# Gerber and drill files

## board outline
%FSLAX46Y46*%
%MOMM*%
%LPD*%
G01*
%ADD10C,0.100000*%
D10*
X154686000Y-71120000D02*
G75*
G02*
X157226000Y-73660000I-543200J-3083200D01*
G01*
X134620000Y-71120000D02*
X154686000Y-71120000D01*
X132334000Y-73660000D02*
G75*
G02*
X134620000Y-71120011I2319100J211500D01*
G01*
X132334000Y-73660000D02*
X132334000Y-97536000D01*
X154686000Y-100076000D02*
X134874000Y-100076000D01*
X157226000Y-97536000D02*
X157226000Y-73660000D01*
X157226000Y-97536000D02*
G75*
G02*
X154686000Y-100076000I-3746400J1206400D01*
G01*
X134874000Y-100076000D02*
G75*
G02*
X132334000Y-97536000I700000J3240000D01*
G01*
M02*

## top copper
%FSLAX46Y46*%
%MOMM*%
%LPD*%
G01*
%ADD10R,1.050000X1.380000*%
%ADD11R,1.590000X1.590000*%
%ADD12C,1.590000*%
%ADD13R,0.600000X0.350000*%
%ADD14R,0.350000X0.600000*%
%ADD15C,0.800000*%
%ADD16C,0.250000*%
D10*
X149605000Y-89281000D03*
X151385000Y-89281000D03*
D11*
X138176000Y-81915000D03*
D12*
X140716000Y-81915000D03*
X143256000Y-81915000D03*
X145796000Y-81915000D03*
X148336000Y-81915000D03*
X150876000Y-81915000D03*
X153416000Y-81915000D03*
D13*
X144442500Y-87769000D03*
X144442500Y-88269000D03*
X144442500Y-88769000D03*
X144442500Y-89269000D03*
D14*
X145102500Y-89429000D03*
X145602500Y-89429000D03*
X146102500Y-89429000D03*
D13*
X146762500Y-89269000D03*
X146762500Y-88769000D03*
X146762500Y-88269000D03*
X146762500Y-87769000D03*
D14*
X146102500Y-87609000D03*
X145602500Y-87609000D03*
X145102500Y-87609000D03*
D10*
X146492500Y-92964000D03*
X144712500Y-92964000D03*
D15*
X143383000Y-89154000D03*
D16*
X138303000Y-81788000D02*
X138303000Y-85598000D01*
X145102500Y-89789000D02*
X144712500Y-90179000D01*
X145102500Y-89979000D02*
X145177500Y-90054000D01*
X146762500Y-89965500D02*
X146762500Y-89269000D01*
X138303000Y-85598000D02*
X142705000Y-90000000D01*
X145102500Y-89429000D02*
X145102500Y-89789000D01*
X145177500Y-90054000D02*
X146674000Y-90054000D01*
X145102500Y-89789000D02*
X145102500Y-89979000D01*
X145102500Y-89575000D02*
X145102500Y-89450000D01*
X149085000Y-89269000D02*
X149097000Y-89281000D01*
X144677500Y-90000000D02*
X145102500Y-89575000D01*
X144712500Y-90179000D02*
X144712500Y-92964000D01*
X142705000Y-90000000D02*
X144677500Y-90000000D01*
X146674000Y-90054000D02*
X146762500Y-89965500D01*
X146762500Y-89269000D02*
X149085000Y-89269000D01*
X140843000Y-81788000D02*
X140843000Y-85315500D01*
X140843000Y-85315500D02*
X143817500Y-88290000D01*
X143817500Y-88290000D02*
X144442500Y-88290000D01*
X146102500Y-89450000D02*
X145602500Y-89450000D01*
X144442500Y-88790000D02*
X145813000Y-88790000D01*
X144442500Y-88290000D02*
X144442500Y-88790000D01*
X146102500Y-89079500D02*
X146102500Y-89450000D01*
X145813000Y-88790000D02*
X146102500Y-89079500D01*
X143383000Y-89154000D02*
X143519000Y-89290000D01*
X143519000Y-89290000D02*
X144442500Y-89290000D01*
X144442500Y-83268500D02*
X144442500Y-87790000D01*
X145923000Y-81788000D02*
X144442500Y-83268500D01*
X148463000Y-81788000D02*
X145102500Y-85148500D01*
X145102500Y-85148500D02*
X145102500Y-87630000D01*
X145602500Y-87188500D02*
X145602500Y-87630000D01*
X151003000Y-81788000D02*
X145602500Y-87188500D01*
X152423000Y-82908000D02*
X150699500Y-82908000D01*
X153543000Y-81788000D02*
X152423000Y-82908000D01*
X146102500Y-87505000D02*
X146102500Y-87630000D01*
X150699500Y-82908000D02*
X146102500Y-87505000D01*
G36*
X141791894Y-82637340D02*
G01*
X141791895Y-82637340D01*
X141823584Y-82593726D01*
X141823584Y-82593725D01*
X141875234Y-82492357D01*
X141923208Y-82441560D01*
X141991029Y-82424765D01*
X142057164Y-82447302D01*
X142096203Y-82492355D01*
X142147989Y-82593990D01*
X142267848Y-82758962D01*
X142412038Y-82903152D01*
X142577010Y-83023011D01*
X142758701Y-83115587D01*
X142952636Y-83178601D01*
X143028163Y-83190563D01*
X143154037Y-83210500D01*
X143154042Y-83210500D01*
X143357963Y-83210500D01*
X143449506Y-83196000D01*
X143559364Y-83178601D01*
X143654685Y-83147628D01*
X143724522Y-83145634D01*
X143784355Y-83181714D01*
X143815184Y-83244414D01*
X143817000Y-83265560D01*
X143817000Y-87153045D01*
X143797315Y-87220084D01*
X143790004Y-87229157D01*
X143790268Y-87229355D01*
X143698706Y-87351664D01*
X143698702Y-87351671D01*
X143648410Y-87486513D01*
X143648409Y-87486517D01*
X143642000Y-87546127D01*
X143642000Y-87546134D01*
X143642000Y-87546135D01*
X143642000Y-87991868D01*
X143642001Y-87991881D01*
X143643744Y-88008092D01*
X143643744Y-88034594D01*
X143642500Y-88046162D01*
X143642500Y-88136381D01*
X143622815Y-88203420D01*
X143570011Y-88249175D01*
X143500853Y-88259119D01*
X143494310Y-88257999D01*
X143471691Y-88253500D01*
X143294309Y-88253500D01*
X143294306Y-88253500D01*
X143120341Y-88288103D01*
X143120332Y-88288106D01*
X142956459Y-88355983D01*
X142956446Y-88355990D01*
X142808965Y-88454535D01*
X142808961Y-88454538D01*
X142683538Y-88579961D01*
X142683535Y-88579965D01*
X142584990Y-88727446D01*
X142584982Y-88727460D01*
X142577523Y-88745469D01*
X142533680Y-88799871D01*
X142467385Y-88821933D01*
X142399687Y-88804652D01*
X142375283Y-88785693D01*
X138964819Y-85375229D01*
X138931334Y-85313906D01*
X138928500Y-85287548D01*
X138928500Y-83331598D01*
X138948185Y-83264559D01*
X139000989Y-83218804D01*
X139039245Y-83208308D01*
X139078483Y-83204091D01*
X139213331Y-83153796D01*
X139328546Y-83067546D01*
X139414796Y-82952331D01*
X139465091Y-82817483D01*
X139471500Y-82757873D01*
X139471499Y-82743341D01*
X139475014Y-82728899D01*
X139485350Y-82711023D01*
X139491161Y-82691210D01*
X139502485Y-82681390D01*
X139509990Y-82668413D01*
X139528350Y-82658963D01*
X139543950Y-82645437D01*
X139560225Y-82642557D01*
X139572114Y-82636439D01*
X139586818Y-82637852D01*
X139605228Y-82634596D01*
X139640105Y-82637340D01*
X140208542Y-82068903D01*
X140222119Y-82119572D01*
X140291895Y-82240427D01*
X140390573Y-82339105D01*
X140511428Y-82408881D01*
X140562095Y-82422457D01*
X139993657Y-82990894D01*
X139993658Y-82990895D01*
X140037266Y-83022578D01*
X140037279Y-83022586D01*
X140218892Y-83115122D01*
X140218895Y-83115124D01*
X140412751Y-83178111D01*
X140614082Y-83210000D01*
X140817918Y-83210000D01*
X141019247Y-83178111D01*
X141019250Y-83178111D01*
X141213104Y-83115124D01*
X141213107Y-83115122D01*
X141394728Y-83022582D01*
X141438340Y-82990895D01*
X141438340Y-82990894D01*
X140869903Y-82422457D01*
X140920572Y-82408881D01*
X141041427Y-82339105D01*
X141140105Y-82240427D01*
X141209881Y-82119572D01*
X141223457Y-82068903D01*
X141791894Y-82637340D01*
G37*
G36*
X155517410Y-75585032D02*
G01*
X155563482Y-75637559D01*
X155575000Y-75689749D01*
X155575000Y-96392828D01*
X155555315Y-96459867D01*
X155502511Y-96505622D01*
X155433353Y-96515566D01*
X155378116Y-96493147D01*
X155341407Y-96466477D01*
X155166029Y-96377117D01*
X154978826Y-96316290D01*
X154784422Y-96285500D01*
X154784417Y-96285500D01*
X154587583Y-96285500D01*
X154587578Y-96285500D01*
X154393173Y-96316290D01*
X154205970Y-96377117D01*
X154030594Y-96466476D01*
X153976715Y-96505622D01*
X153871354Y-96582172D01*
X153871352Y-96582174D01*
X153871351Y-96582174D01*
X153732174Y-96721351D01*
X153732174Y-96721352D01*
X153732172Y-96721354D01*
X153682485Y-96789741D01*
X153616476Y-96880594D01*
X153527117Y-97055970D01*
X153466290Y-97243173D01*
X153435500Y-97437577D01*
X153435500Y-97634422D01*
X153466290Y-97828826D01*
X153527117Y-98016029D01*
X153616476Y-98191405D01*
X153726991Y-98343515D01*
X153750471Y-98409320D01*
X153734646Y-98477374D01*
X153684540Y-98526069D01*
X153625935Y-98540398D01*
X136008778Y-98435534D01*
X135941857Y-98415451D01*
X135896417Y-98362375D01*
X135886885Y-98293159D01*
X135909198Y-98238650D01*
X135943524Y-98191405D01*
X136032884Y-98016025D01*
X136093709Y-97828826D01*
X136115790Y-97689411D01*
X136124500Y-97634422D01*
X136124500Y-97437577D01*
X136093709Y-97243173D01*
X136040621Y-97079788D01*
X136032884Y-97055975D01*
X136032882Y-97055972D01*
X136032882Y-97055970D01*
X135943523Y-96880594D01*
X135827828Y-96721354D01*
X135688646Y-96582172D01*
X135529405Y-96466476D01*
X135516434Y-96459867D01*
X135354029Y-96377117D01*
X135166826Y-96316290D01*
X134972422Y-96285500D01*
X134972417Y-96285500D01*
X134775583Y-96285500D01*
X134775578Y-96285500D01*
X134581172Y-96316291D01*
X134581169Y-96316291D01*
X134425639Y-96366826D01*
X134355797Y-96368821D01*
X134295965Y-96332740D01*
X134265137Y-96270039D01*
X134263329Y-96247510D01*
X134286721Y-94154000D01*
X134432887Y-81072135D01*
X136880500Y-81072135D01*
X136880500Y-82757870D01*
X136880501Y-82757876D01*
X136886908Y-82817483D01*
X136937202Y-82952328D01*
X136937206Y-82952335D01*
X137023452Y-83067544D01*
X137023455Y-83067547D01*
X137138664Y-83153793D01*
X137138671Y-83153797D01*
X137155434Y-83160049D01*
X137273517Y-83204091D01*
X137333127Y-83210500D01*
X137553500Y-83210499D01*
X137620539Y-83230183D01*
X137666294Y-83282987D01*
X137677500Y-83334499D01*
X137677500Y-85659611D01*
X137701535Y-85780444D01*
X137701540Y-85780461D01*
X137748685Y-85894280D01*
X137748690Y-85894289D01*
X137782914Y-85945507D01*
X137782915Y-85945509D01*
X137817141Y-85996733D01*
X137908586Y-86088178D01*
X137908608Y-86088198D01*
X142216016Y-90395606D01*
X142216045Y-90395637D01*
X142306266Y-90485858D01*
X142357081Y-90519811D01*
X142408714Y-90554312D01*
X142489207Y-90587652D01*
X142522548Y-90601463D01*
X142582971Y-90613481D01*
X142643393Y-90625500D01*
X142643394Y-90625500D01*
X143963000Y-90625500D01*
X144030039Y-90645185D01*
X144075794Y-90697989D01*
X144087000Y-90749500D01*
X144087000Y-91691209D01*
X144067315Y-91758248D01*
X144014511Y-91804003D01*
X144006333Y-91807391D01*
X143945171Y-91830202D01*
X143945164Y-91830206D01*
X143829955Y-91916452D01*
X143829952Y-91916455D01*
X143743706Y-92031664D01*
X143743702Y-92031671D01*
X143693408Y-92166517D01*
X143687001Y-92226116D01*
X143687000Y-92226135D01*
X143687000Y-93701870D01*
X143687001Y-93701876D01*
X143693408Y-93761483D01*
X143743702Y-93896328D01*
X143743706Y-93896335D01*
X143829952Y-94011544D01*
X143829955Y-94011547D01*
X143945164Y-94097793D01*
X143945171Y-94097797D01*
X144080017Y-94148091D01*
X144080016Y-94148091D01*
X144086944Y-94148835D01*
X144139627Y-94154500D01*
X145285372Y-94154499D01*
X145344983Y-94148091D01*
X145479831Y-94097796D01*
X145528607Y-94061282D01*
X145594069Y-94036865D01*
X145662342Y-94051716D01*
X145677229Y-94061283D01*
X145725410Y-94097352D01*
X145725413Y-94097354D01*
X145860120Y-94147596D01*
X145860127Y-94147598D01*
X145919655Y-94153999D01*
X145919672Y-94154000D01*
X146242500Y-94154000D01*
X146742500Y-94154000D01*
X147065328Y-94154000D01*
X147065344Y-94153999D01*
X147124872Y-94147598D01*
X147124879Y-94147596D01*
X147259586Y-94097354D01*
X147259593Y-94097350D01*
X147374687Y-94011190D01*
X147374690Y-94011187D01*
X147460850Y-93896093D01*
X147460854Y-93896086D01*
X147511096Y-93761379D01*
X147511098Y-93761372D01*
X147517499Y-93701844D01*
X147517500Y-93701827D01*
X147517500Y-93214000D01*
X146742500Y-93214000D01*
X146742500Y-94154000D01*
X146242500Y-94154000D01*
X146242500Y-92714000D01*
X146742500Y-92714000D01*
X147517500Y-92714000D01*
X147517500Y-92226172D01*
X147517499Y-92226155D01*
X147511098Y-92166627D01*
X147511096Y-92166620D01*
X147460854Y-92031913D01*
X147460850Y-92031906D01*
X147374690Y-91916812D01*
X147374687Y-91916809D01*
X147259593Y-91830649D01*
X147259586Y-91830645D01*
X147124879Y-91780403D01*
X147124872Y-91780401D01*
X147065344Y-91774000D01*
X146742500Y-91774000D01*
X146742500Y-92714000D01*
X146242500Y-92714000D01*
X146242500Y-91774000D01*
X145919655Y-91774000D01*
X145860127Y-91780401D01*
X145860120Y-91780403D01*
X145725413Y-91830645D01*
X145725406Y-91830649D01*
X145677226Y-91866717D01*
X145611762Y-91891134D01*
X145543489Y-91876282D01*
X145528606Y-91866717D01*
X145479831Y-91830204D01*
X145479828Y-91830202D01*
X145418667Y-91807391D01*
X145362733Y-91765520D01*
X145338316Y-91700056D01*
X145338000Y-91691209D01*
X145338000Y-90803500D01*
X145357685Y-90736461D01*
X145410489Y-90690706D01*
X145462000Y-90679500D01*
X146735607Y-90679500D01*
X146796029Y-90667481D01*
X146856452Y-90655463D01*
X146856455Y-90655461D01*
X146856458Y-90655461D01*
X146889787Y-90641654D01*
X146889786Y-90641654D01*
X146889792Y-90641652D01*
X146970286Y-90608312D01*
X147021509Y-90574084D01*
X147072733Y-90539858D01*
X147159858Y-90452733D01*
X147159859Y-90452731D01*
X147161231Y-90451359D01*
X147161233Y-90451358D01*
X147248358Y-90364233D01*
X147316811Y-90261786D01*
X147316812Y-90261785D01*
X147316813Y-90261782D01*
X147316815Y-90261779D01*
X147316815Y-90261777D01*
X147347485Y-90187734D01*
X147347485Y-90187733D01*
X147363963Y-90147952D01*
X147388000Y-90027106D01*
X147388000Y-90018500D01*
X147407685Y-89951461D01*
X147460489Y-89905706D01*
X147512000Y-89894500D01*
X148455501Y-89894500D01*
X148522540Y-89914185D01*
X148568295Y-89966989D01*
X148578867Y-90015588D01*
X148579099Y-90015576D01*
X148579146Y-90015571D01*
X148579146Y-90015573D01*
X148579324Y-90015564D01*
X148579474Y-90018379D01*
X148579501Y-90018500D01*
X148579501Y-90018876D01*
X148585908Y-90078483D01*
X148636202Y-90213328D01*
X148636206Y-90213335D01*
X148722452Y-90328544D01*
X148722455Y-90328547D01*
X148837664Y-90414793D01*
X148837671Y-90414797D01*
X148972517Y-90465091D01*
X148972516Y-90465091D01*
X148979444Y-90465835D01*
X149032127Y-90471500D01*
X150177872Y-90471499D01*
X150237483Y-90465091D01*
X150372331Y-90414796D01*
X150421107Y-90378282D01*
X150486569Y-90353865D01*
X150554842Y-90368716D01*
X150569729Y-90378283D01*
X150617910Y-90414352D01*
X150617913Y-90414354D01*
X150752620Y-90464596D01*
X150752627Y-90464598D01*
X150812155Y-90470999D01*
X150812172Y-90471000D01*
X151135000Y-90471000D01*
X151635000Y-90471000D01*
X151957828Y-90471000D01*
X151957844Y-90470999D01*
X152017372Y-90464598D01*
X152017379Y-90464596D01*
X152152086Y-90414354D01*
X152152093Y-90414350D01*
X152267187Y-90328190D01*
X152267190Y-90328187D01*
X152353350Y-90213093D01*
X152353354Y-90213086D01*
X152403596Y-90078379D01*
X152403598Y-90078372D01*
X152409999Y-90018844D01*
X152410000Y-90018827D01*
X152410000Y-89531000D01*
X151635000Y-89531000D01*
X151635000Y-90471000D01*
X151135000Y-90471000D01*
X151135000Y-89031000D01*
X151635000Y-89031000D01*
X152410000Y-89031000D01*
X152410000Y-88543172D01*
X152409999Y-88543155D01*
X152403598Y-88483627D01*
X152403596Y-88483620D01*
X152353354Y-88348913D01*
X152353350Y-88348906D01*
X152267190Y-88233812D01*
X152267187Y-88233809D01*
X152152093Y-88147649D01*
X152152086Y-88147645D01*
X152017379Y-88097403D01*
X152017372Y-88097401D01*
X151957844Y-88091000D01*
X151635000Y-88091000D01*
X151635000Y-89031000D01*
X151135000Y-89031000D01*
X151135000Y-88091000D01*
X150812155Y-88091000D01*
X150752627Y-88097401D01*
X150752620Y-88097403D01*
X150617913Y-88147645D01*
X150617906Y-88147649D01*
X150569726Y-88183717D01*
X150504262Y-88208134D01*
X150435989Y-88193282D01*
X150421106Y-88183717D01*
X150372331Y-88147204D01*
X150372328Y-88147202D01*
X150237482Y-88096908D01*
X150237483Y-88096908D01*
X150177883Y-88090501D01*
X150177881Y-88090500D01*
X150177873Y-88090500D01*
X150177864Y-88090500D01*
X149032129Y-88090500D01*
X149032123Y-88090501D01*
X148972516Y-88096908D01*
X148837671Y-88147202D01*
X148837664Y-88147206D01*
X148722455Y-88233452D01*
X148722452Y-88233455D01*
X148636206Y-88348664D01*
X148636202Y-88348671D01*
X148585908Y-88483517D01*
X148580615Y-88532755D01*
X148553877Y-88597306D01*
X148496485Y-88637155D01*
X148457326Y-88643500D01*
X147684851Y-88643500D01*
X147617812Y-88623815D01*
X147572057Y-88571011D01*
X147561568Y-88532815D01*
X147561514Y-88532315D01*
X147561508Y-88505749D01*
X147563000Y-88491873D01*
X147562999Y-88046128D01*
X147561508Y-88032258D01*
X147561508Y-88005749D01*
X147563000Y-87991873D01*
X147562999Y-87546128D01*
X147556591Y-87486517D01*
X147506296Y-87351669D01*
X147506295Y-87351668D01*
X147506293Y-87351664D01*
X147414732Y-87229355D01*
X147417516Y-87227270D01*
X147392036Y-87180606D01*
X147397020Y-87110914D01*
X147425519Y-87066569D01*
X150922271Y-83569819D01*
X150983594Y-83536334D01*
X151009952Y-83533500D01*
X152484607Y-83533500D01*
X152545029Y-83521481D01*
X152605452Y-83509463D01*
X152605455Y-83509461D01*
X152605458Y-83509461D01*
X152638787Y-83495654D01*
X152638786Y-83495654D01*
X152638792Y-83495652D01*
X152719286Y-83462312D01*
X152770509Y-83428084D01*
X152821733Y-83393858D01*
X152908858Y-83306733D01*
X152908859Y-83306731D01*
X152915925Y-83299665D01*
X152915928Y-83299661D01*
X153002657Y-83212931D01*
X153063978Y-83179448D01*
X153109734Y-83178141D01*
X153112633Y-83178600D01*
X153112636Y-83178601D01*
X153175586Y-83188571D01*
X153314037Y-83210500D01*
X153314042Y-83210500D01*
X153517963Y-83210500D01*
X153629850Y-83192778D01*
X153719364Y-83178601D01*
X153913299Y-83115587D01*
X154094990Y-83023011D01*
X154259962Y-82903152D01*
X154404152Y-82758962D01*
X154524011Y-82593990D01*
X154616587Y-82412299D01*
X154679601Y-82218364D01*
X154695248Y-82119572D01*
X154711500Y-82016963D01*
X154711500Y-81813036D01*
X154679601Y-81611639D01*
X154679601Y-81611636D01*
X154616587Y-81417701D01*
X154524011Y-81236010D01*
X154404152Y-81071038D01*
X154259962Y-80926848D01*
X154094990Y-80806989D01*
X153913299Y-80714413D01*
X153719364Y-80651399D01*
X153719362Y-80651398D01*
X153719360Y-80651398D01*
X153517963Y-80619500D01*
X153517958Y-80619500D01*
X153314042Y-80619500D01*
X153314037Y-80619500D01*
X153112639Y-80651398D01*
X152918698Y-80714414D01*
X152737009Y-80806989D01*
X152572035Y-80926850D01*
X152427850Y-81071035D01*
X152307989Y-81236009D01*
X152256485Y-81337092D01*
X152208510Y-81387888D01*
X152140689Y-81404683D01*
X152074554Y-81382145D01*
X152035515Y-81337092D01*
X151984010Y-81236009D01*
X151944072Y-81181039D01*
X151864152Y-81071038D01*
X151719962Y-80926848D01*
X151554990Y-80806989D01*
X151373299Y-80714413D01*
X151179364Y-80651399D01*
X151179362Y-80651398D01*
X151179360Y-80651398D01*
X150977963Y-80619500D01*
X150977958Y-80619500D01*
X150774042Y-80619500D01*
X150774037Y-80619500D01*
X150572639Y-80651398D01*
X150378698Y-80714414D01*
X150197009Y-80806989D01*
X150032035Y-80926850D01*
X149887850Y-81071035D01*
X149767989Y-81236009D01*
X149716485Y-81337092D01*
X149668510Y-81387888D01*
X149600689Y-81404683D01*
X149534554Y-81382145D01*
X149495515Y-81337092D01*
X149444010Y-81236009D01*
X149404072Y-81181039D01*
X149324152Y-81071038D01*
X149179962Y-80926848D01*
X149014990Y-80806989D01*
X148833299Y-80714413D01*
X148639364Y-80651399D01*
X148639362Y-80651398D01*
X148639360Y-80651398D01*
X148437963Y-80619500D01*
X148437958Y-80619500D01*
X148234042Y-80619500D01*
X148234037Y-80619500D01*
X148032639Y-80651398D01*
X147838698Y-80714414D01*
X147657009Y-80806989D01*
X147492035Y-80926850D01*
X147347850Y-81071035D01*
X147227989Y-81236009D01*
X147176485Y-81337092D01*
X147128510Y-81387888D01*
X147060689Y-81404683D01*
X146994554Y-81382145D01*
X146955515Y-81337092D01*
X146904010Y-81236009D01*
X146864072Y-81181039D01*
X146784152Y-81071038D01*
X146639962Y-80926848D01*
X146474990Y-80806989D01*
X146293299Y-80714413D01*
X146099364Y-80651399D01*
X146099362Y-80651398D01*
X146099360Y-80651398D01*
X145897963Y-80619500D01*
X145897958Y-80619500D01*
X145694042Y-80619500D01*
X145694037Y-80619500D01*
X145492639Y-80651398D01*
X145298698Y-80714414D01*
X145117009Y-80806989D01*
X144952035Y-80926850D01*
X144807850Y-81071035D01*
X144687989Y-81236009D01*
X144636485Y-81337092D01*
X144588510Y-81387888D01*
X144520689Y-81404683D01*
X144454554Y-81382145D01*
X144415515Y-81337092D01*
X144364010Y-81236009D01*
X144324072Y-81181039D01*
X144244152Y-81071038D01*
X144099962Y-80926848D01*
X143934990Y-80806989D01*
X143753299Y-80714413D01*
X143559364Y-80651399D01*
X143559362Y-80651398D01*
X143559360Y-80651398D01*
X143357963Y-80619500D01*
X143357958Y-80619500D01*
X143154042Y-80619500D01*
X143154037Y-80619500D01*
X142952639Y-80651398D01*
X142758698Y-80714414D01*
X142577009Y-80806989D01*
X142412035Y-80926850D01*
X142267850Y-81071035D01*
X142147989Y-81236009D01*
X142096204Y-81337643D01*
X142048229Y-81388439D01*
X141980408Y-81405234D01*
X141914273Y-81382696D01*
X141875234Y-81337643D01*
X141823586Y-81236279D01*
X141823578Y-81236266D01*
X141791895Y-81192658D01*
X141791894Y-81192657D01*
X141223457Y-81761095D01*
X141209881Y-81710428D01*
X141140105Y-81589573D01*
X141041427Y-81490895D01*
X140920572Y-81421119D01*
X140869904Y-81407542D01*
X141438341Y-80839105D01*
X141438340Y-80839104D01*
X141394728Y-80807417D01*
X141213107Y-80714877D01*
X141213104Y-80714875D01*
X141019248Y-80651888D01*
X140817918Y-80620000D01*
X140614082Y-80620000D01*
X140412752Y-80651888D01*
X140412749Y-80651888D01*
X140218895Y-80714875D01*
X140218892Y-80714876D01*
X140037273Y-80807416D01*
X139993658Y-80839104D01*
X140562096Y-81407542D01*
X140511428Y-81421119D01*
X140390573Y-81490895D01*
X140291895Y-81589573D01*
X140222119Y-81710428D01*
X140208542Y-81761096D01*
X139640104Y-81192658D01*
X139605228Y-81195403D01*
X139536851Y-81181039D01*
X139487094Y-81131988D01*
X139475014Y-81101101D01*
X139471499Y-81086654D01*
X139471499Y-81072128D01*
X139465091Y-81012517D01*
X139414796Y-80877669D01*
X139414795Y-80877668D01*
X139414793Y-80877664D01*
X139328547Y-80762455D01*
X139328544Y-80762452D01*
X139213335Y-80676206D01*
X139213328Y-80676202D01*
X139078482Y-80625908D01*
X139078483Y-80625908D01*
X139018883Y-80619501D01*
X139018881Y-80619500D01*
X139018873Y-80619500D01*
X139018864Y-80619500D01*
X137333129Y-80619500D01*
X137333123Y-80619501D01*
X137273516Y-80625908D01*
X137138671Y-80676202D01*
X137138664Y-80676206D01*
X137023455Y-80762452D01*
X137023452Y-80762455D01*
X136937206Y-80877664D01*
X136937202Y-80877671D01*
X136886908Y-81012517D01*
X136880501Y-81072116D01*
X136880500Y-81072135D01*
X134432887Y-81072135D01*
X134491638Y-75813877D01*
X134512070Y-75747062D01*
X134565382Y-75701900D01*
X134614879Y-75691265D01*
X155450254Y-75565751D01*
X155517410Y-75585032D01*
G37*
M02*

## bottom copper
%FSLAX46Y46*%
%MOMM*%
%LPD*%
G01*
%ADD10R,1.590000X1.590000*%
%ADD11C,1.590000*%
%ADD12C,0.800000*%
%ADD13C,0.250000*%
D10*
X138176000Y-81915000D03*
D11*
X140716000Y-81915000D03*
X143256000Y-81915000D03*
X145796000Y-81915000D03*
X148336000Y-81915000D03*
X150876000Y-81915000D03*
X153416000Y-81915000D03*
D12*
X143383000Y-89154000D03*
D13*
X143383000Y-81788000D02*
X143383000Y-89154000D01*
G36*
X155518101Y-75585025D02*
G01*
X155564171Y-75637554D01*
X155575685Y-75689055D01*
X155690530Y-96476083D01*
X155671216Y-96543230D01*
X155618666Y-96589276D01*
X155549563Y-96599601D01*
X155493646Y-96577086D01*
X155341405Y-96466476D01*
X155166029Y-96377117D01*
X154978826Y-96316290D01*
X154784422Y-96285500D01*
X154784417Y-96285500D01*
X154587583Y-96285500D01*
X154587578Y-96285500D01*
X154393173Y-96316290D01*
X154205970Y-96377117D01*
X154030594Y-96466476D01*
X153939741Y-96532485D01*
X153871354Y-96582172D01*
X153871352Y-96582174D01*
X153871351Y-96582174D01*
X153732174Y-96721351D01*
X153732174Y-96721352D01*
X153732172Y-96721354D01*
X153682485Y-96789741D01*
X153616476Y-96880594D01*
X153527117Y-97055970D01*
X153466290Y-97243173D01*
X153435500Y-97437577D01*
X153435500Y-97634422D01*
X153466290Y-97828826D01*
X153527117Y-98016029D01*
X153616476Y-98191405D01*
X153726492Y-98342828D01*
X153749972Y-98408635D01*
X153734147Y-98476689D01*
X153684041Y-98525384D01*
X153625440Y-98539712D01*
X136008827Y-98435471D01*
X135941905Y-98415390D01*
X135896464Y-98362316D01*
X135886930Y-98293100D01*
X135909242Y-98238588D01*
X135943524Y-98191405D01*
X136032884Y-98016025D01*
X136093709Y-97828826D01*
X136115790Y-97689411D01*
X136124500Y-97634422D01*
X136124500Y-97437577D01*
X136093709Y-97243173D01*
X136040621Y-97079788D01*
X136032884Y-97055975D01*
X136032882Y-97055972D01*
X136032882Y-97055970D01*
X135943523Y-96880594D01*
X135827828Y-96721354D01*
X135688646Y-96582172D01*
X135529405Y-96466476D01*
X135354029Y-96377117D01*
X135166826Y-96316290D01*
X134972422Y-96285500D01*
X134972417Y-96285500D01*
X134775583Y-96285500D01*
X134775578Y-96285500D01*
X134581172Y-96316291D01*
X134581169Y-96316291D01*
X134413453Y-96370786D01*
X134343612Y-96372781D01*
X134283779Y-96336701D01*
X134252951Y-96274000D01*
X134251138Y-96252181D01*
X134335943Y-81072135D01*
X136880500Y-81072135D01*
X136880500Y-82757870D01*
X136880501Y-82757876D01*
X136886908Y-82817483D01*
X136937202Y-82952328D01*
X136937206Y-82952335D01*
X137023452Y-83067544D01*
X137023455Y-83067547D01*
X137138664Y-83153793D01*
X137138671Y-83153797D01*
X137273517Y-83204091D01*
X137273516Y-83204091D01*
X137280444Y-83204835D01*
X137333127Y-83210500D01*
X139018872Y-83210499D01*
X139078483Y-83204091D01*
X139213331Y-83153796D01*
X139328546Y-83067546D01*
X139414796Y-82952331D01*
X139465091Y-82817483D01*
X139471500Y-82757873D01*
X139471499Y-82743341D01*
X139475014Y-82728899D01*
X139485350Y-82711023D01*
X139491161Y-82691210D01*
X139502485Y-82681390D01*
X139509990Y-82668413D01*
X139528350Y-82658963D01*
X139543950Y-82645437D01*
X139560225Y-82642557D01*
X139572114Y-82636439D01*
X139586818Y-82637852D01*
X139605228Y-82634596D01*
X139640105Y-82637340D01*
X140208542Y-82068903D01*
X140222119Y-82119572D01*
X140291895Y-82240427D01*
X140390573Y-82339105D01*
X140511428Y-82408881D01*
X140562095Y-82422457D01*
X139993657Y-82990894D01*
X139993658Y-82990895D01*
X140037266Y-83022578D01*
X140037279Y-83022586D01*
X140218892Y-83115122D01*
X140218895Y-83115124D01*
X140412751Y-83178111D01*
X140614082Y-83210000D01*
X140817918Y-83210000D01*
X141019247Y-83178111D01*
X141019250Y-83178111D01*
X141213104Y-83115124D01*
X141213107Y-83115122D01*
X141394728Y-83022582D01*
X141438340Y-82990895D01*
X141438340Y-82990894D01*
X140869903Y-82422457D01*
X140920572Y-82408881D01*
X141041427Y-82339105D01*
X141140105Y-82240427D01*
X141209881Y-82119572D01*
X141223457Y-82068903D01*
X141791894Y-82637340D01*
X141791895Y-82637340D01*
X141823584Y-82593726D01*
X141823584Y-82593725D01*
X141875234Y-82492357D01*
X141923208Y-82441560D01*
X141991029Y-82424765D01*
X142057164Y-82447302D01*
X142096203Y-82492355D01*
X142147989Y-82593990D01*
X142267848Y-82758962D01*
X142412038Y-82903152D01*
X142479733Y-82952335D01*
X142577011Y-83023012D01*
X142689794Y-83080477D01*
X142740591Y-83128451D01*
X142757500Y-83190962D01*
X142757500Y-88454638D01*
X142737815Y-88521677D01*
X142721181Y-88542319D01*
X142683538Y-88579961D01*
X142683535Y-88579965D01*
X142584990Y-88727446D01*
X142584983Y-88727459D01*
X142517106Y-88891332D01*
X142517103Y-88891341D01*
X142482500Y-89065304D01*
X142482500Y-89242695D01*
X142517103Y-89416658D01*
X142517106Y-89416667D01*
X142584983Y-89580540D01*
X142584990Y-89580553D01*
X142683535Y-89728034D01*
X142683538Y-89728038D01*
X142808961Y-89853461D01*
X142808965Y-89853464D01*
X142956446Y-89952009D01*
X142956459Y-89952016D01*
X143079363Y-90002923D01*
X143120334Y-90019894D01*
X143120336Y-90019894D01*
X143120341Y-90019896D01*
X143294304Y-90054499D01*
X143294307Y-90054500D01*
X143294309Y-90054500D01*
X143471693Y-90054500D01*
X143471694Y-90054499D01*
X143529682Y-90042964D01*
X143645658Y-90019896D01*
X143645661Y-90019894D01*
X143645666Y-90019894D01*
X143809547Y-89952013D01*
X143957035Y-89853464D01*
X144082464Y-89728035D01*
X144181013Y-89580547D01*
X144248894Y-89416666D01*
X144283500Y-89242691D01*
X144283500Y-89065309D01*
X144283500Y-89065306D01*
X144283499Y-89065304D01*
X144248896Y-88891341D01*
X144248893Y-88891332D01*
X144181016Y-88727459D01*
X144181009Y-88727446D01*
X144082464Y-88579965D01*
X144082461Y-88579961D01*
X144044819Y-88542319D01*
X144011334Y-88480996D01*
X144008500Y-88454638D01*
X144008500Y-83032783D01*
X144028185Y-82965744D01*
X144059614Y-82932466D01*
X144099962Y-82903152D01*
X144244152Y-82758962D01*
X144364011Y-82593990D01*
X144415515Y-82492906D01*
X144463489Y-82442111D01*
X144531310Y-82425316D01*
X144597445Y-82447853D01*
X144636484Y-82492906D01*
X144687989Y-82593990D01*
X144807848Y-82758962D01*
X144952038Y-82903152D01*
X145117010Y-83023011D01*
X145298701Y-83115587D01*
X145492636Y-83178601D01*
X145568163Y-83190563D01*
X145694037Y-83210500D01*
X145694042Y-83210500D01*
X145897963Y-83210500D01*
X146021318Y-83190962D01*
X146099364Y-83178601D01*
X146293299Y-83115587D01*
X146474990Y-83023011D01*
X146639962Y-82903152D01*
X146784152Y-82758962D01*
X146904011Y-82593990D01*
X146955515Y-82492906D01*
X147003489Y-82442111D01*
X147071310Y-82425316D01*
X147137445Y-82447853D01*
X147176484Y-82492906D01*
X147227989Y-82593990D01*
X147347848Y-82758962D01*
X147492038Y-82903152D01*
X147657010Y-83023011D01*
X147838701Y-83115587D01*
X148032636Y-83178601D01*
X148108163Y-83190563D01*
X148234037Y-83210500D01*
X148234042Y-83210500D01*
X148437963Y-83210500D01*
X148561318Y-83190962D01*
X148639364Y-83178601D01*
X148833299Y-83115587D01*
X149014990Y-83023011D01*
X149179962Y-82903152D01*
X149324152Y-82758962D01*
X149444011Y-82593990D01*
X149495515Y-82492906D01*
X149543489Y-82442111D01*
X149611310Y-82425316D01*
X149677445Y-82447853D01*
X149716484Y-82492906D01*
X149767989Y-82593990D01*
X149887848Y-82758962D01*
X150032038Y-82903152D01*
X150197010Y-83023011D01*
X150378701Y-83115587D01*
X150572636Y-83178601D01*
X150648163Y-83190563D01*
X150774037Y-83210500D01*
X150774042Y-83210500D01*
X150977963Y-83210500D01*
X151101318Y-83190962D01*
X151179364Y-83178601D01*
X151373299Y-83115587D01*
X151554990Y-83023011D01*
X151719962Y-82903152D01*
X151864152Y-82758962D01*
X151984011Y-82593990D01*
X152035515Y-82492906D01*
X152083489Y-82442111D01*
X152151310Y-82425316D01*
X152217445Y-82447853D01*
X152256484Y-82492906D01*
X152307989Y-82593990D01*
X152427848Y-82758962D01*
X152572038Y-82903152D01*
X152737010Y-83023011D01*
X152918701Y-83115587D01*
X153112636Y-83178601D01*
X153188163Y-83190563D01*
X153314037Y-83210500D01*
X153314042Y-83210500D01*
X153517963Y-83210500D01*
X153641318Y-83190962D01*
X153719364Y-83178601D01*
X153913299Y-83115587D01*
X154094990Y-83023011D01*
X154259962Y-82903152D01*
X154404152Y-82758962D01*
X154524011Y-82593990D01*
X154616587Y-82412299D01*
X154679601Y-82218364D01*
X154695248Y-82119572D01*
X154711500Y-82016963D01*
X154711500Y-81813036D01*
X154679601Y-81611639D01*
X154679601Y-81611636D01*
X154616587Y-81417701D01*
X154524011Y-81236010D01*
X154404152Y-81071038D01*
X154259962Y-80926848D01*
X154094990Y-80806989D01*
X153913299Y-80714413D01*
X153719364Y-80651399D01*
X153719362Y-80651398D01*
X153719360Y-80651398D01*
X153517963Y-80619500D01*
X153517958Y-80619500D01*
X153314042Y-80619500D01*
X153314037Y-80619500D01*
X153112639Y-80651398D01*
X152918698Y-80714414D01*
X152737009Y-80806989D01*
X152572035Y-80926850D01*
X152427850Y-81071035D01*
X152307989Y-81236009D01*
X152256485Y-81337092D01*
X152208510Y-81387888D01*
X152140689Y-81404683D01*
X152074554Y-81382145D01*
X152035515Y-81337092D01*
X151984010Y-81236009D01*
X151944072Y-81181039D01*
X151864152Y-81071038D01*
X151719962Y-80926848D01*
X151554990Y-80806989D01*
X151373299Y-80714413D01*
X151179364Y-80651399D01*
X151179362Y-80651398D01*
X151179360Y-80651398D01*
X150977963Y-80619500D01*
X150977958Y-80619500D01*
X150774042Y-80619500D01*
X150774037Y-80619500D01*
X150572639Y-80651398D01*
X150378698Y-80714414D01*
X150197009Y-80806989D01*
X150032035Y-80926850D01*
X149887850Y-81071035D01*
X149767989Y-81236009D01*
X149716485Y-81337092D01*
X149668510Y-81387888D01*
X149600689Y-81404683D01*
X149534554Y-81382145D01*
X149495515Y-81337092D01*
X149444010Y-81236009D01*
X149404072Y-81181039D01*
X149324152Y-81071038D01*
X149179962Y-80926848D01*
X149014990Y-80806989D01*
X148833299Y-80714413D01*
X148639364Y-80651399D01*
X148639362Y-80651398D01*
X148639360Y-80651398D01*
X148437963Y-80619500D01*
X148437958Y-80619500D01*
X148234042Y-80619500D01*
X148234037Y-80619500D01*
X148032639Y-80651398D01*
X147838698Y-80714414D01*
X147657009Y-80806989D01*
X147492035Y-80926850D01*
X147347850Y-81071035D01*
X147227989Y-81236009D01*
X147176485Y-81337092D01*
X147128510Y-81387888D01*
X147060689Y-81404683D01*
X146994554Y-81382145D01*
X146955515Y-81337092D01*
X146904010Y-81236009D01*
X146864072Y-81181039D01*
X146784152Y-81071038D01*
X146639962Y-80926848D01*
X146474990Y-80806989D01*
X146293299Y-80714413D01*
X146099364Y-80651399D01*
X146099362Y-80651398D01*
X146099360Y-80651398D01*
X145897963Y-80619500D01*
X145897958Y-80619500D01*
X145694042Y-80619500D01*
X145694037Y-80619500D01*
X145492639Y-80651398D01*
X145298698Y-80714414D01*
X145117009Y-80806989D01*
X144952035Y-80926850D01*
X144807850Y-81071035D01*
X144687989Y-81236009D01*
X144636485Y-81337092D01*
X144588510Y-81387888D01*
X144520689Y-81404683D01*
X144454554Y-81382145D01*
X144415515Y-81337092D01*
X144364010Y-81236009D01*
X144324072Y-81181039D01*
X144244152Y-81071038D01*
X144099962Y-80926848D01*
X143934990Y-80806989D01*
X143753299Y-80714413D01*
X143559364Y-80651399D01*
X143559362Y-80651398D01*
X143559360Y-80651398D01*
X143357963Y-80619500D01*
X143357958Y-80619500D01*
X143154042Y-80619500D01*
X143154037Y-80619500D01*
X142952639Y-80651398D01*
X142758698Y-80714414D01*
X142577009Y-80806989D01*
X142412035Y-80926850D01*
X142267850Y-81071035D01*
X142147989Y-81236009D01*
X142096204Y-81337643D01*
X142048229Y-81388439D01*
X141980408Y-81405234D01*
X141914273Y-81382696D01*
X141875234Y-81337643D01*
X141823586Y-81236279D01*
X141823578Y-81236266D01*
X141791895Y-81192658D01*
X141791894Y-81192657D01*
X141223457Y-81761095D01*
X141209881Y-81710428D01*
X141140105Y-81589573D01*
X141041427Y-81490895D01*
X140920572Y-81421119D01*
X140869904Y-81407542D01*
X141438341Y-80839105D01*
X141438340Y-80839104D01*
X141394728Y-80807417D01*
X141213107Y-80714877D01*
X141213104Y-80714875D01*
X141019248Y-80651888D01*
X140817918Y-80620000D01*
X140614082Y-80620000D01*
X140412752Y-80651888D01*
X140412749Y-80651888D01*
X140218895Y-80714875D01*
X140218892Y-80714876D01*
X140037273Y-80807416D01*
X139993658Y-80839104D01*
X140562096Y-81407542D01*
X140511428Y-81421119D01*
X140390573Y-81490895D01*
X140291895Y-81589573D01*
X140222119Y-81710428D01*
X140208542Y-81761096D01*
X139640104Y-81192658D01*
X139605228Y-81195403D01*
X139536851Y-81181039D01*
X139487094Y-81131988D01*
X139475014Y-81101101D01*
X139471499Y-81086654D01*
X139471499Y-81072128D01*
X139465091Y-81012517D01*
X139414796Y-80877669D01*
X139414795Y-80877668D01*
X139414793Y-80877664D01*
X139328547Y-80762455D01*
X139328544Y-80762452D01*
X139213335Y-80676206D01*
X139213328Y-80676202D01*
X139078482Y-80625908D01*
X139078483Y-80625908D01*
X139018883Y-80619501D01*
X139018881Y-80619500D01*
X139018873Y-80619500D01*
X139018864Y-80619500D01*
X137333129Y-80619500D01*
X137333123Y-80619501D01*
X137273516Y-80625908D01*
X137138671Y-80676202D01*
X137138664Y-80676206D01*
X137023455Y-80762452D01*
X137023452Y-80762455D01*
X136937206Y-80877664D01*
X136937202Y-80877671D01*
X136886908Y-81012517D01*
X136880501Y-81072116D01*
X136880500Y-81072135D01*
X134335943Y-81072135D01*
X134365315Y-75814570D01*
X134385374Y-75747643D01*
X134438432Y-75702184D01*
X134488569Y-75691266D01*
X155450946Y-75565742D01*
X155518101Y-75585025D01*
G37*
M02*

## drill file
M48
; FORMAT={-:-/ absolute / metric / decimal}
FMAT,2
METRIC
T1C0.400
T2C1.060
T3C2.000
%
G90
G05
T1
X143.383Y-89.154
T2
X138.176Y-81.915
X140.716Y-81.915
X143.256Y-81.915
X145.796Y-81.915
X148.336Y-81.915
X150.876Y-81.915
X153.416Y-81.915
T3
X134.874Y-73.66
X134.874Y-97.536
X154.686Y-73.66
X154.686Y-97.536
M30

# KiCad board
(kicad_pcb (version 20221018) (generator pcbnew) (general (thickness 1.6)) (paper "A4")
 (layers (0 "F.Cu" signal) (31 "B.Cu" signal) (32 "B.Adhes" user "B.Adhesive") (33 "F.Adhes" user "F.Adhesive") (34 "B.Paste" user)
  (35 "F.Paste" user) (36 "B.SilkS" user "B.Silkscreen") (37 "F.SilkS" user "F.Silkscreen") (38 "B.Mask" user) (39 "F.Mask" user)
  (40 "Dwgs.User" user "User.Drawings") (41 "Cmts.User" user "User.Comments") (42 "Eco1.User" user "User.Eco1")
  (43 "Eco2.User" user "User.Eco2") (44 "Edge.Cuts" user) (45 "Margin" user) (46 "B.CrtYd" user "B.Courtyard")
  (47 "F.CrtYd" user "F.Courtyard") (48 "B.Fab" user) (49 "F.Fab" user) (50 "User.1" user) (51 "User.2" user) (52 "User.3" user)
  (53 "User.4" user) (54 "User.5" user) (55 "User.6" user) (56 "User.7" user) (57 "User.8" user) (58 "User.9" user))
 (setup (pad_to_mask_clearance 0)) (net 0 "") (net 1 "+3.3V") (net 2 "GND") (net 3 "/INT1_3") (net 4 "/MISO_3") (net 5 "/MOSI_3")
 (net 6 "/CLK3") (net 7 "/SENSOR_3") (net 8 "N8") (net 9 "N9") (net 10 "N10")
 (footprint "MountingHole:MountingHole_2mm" (layer "F.Cu") (at 134.874 97.536)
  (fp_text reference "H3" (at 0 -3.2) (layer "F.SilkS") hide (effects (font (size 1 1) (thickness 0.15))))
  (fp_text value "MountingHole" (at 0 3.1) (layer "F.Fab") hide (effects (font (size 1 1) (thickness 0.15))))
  (pad "" np_thru_hole circle (at 0 0) (size 2 2) (drill 2) (layers "*.Cu" "*.Mask")))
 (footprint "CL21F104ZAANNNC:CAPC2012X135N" (layer "F.Cu") (at 150.495 89.281)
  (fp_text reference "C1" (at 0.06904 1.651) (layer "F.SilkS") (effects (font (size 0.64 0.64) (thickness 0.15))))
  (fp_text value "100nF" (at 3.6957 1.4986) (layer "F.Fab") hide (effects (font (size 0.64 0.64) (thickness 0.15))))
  (pad "1" smd rect (at -0.89 0) (size 1.05 1.38) (layers "F.Cu" "F.Paste" "F.Mask") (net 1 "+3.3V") (solder_mask_margin 0.102))
  (pad "2" smd rect (at 0.89 0) (size 1.05 1.38) (layers "F.Cu" "F.Paste" "F.Mask") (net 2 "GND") (solder_mask_margin 0.102)))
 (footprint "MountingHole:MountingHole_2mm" (layer "F.Cu") (at 154.686 73.66)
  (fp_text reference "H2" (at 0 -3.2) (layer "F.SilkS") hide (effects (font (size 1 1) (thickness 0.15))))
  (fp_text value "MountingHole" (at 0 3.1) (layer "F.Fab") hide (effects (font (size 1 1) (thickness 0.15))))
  (pad "" np_thru_hole circle (at 0 0) (size 2 2) (drill 2) (layers "*.Cu" "*.Mask")))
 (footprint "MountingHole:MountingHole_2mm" (layer "F.Cu") (at 134.874 73.66)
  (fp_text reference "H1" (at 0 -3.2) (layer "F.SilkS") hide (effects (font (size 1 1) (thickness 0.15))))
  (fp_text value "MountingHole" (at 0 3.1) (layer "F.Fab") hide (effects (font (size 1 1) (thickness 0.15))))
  (pad "" np_thru_hole circle (at 0 0) (size 2 2) (drill 2) (layers "*.Cu" "*.Mask")))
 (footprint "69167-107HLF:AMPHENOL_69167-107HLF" (layer "F.Cu") (at 145.796 81.915)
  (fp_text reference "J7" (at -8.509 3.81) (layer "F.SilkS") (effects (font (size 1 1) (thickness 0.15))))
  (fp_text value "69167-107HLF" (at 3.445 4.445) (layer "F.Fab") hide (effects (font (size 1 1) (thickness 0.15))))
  (pad "01" thru_hole rect (at -7.62 0) (size 1.59 1.59) (drill 1.06) (layers "*.Cu" "*.Mask") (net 1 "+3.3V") (solder_mask_margin 0.102))
  (pad "02" thru_hole circle (at -5.08 0) (size 1.59 1.59) (drill 1.06) (layers "*.Cu" "*.Mask") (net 2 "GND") (solder_mask_margin 0.102))
  (pad "03" thru_hole circle (at -2.54 0) (size 1.59 1.59) (drill 1.06) (layers "*.Cu" "*.Mask") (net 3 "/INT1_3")
   (solder_mask_margin 0.102))
  (pad "04" thru_hole circle (at 0 0) (size 1.59 1.59) (drill 1.06) (layers "*.Cu" "*.Mask") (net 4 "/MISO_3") (solder_mask_margin 0.102))
  (pad "05" thru_hole circle (at 2.54 0) (size 1.59 1.59) (drill 1.06) (layers "*.Cu" "*.Mask") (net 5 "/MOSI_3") (solder_mask_margin 0.102))
  (pad "06" thru_hole circle (at 5.08 0) (size 1.59 1.59) (drill 1.06) (layers "*.Cu" "*.Mask") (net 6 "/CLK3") (solder_mask_margin 0.102))
  (pad "07" thru_hole circle (at 7.62 0) (size 1.59 1.59) (drill 1.06) (layers "*.Cu" "*.Mask") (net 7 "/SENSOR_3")
   (solder_mask_margin 0.102)))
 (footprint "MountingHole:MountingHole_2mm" (layer "F.Cu") (at 154.686 97.536)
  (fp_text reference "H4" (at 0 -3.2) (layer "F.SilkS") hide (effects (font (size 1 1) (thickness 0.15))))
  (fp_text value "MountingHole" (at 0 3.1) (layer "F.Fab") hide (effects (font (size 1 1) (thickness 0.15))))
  (pad "" np_thru_hole circle (at 0 0) (size 2 2) (drill 2) (layers "*.Cu" "*.Mask")))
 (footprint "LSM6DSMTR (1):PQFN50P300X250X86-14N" (layer "F.Cu") (at 145.6025 88.519)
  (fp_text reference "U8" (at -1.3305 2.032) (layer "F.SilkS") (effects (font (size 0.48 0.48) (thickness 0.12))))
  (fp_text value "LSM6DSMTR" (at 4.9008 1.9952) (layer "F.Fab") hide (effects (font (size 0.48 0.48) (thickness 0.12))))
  (pad "1" smd rect (at -1.16 -0.75) (size 0.6 0.35) (layers "F.Cu" "F.Paste" "F.Mask") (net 4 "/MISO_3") (solder_mask_margin 0.102))
  (pad "2" smd rect (at -1.16 -0.25) (size 0.6 0.35) (layers "F.Cu" "F.Paste" "F.Mask") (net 2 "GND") (solder_mask_margin 0.102))
  (pad "3" smd rect (at -1.16 0.25) (size 0.6 0.35) (layers "F.Cu" "F.Paste" "F.Mask") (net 2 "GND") (solder_mask_margin 0.102))
  (pad "4" smd rect (at -1.16 0.75) (size 0.6 0.35) (layers "F.Cu" "F.Paste" "F.Mask") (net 3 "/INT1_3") (solder_mask_margin 0.102))
  (pad "5" smd rect (at -0.5 0.91 90) (size 0.6 0.35) (layers "F.Cu" "F.Paste" "F.Mask") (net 1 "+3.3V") (solder_mask_margin 0.102))
  (pad "6" smd rect (at 0 0.91 90) (size 0.6 0.35) (layers "F.Cu" "F.Paste" "F.Mask") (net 2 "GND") (solder_mask_margin 0.102))
  (pad "7" smd rect (at 0.5 0.91 90) (size 0.6 0.35) (layers "F.Cu" "F.Paste" "F.Mask") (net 2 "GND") (solder_mask_margin 0.102))
  (pad "8" smd rect (at 1.16 0.75) (size 0.6 0.35) (layers "F.Cu" "F.Paste" "F.Mask") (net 1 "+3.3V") (solder_mask_margin 0.102))
  (pad "9" smd rect (at 1.16 0.25) (size 0.6 0.35) (layers "F.Cu" "F.Paste" "F.Mask") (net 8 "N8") (solder_mask_margin 0.102))
  (pad "10" smd rect (at 1.16 -0.25) (size 0.6 0.35) (layers "F.Cu" "F.Paste" "F.Mask") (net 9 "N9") (solder_mask_margin 0.102))
  (pad "11" smd rect (at 1.16 -0.75) (size 0.6 0.35) (layers "F.Cu" "F.Paste" "F.Mask") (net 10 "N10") (solder_mask_margin 0.102))
  (pad "12" smd rect (at 0.5 -0.91 90) (size 0.6 0.35) (layers "F.Cu" "F.Paste" "F.Mask") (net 7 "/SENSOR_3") (solder_mask_margin 0.102))
  (pad "13" smd rect (at 0 -0.91 90) (size 0.6 0.35) (layers "F.Cu" "F.Paste" "F.Mask") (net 6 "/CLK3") (solder_mask_margin 0.102))
  (pad "14" smd rect (at -0.5 -0.91 90) (size 0.6 0.35) (layers "F.Cu" "F.Paste" "F.Mask") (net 5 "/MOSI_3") (solder_mask_margin 0.102)))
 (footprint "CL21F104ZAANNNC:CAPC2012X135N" (layer "F.Cu") (at 145.6025 92.964 180)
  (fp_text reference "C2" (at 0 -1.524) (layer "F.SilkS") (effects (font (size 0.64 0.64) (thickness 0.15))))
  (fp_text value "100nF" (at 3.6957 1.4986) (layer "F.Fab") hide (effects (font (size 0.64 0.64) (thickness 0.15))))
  (pad "1" smd rect (at -0.89 0 180) (size 1.05 1.38) (layers "F.Cu" "F.Paste" "F.Mask") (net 2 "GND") (solder_mask_margin 0.102))
  (pad "2" smd rect (at 0.89 0 180) (size 1.05 1.38) (layers "F.Cu" "F.Paste" "F.Mask") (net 1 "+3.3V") (solder_mask_margin 0.102)))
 (gr_arc (start 154.686 71.12) (mid 156.356529 71.989471) (end 157.226 73.66) (stroke (width 0.1) (type default)) (layer "Edge.Cuts"))
 (gr_line (start 134.62 71.12) (end 154.686 71.12) (stroke (width 0.1) (type default)) (layer "Edge.Cuts"))
 (gr_arc (start 132.334 73.66) (mid 132.922178 71.89066) (end 134.62 71.12) (stroke (width 0.1) (type default)) (layer "Edge.Cuts"))
 (gr_line (start 132.334 73.66) (end 132.334 97.536) (stroke (width 0.1) (type default)) (layer "Edge.Cuts"))
 (gr_line (start 154.686 100.076) (end 134.874 100.076) (stroke (width 0.1) (type default)) (layer "Edge.Cuts"))
 (gr_line (start 157.226 97.536) (end 157.226 73.66) (stroke (width 0.1) (type default)) (layer "Edge.Cuts"))
 (gr_arc (start 157.226 97.536) (mid 156.262666 99.112666) (end 154.686 100.076) (stroke (width 0.1) (type default)) (layer "Edge.Cuts"))
 (gr_arc (start 134.874 100.076) (mid 133.230114 99.179886) (end 132.334 97.536) (stroke (width 0.1) (type default)) (layer "Edge.Cuts"))
 (segment (start 138.303 81.788) (end 138.303 85.598) (width 0.25) (layer "F.Cu") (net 1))
 (segment (start 145.1025 89.789) (end 144.7125 90.179) (width 0.25) (layer "F.Cu") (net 1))
 (segment (start 145.1025 89.979) (end 145.1775 90.054) (width 0.25) (layer "F.Cu") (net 1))
 (segment (start 146.7625 89.9655) (end 146.7625 89.269) (width 0.25) (layer "F.Cu") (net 1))
 (segment (start 138.303 85.598) (end 142.705 90) (width 0.25) (layer "F.Cu") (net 1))
 (segment (start 145.1025 89.429) (end 145.1025 89.789) (width 0.25) (layer "F.Cu") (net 1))
 (segment (start 145.1775 90.054) (end 146.674 90.054) (width 0.25) (layer "F.Cu") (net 1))
 (segment (start 145.1025 89.789) (end 145.1025 89.979) (width 0.25) (layer "F.Cu") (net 1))
 (segment (start 145.1025 89.575) (end 145.1025 89.45) (width 0.25) (layer "F.Cu") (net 1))
 (segment (start 149.085 89.269) (end 149.097 89.281) (width 0.25) (layer "F.Cu") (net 1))
 (segment (start 144.6775 90) (end 145.1025 89.575) (width 0.25) (layer "F.Cu") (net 1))
 (segment (start 144.7125 90.179) (end 144.7125 92.964) (width 0.25) (layer "F.Cu") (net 1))
 (segment (start 142.705 90) (end 144.6775 90) (width 0.25) (layer "F.Cu") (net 1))
 (segment (start 146.674 90.054) (end 146.7625 89.9655) (width 0.25) (layer "F.Cu") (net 1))
 (segment (start 146.7625 89.269) (end 149.085 89.269) (width 0.25) (layer "F.Cu") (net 1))
 (segment (start 140.843 81.788) (end 140.843 85.3155) (width 0.25) (layer "F.Cu") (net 2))
 (segment (start 140.843 85.3155) (end 143.8175 88.29) (width 0.25) (layer "F.Cu") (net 2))
 (segment (start 143.8175 88.29) (end 144.4425 88.29) (width 0.25) (layer "F.Cu") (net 2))
 (segment (start 146.1025 89.45) (end 145.6025 89.45) (width 0.25) (layer "F.Cu") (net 2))
 (segment (start 144.4425 88.79) (end 145.813 88.79) (width 0.25) (layer "F.Cu") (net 2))
 (segment (start 144.4425 88.29) (end 144.4425 88.79) (width 0.25) (layer "F.Cu") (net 2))
 (segment (start 146.1025 89.0795) (end 146.1025 89.45) (width 0.25) (layer "F.Cu") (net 2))
 (segment (start 145.813 88.79) (end 146.1025 89.0795) (width 0.25) (layer "F.Cu") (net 2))
 (segment (start 143.383 89.154) (end 143.519 89.29) (width 0.25) (layer "F.Cu") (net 3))
 (segment (start 143.519 89.29) (end 144.4425 89.29) (width 0.25) (layer "F.Cu") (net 3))
 (via (at 143.383 89.154) (size 0.8) (drill 0.4) (layers "F.Cu" "B.Cu") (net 3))
 (segment (start 143.383 81.788) (end 143.383 89.154) (width 0.25) (layer "B.Cu") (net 3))
 (segment (start 144.4425 83.2685) (end 144.4425 87.79) (width 0.25) (layer "F.Cu") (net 4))
 (segment (start 145.923 81.788) (end 144.4425 83.2685) (width 0.25) (layer "F.Cu") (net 4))
 (segment (start 148.463 81.788) (end 145.1025 85.1485) (width 0.25) (layer "F.Cu") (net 5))
 (segment (start 145.1025 85.1485) (end 145.1025 87.63) (width 0.25) (layer "F.Cu") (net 5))
 (segment (start 145.6025 87.1885) (end 145.6025 87.63) (width 0.25) (layer "F.Cu") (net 6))
 (segment (start 151.003 81.788) (end 145.6025 87.1885) (width 0.25) (layer "F.Cu") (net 6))
 (segment (start 152.423 82.908) (end 150.6995 82.908) (width 0.25) (layer "F.Cu") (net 7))
 (segment (start 153.543 81.788) (end 152.423 82.908) (width 0.25) (layer "F.Cu") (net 7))
 (segment (start 146.1025 87.505) (end 146.1025 87.63) (width 0.25) (layer "F.Cu") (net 7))
 (segment (start 150.6995 82.908) (end 146.1025 87.505) (width 0.25) (layer "F.Cu") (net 7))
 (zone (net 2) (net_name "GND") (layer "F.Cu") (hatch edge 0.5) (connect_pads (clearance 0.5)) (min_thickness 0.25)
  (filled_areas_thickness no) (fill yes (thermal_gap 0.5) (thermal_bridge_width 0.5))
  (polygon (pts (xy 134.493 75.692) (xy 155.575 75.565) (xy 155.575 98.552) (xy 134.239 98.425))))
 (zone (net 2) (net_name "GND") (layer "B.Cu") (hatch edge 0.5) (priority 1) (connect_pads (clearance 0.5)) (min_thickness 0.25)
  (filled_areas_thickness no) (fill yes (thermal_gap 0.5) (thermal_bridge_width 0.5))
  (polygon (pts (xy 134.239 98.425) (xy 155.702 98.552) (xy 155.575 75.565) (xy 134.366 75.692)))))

